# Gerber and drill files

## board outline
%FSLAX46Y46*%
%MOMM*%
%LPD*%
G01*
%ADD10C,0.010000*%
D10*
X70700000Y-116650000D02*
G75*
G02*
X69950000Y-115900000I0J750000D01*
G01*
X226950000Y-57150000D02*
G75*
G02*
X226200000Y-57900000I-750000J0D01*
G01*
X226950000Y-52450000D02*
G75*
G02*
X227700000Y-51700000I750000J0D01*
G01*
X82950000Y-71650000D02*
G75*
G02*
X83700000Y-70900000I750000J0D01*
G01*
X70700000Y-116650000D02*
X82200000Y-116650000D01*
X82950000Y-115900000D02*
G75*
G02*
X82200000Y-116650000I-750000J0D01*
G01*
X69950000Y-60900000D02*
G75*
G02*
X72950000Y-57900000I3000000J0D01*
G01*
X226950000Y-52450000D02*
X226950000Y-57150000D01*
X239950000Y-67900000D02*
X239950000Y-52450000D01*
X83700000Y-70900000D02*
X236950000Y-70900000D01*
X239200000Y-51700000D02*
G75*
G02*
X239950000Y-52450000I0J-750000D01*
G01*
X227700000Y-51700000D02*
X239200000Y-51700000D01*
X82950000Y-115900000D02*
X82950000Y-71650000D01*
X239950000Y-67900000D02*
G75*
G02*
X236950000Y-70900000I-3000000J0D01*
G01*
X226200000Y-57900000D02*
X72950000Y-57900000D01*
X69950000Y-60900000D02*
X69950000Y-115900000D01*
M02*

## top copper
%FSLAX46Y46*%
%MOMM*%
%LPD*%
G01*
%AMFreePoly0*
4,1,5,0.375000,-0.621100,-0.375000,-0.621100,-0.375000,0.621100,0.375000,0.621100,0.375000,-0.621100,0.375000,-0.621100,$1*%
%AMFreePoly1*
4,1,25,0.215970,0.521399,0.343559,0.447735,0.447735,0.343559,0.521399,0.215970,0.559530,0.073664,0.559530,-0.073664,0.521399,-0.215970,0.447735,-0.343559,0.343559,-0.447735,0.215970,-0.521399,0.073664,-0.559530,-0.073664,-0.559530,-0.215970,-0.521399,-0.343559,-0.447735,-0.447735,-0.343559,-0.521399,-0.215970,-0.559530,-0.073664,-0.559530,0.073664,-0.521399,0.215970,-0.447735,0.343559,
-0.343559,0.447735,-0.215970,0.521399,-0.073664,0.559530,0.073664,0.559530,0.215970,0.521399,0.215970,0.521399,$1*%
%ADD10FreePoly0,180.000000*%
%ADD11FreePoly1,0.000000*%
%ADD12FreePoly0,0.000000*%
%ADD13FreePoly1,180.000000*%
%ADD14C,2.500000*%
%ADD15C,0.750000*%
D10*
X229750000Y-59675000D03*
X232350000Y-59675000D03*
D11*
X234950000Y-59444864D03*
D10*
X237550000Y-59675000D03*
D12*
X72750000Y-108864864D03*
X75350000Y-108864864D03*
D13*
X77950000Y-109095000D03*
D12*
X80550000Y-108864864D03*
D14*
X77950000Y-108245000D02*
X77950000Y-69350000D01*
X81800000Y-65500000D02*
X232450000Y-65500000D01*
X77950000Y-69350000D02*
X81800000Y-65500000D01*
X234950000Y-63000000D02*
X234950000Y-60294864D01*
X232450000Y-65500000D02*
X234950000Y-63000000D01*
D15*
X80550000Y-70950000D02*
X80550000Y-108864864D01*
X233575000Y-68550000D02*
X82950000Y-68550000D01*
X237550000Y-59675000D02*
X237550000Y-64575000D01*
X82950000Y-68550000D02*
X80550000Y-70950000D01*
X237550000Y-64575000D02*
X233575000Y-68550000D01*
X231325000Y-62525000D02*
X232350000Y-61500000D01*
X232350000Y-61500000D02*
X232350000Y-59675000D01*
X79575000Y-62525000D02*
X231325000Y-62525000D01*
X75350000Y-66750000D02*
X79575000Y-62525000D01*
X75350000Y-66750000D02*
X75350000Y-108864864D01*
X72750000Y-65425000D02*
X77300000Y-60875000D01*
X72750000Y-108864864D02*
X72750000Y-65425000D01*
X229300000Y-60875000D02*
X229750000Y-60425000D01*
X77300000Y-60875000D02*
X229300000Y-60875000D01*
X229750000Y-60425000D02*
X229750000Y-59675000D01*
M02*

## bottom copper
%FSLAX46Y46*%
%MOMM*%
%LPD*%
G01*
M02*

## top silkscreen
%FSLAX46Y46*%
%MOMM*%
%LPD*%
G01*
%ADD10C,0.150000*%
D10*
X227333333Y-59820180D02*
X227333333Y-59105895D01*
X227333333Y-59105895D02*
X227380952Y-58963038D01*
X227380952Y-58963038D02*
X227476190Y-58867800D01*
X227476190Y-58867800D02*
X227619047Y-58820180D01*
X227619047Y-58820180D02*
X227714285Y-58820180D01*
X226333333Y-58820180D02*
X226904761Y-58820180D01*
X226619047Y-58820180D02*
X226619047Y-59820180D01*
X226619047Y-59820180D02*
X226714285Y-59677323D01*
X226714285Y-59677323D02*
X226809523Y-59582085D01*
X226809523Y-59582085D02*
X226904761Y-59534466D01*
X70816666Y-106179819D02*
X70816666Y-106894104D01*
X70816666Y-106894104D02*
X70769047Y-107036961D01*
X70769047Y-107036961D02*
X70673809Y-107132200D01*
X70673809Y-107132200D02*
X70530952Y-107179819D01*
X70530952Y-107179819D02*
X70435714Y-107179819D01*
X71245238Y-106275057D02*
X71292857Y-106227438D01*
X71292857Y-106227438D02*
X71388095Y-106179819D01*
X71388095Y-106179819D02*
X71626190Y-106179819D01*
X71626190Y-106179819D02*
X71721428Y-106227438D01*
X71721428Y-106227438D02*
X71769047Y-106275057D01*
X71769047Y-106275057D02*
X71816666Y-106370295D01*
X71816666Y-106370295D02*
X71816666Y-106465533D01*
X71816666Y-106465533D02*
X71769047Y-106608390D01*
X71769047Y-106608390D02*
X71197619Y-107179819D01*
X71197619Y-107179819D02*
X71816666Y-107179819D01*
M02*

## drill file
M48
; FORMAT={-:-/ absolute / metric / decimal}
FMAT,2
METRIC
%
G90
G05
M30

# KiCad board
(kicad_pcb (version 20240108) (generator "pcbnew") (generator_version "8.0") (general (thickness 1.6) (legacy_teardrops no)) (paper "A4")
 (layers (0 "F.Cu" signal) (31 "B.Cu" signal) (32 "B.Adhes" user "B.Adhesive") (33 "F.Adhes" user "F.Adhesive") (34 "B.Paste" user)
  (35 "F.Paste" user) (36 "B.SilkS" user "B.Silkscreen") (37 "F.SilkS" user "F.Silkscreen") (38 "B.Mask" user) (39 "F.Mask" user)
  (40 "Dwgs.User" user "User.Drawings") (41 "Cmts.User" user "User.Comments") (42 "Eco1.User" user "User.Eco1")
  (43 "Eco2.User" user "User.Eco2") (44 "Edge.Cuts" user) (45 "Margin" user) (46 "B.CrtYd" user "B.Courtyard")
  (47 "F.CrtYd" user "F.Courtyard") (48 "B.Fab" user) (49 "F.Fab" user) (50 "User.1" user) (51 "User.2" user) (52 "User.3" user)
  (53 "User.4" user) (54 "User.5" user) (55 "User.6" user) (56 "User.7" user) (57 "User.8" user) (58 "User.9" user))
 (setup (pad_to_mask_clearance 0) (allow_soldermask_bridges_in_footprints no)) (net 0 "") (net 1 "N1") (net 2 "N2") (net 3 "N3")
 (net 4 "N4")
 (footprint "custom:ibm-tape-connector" (layer "F.Cu") (at 233.45 56.314864 180)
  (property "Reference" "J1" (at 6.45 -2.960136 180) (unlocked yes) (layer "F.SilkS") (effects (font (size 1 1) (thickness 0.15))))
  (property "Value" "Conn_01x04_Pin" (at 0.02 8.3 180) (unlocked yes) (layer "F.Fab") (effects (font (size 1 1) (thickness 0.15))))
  (pad "1" smd custom (at 3.7 -3.360136 180) (size 0.75 1.2422) (layers "F.Cu" "F.Paste" "F.Mask") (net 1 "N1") (thermal_bridge_angle 45)
   (options (clearance outline) (anchor rect)) (primitives))
  (pad "2" smd custom (at 1.1 -3.360136 180) (size 0.75 1.2422) (layers "F.Cu" "F.Paste" "F.Mask") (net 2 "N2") (thermal_bridge_angle 45)
   (options (clearance outline) (anchor rect)) (primitives))
  (pad "3" smd custom (at -1.5 -3.98) (size 1.128716 1.128716) (drill (offset 0 -0.85)) (layers "F.Cu" "F.Paste" "F.Mask") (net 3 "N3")
   (options (clearance outline) (anchor circle)) (primitives))
  (pad "4" smd custom (at -4.1 -3.360136 180) (size 0.75 1.2422) (layers "F.Cu" "F.Paste" "F.Mask") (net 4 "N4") (thermal_bridge_angle 45)
   (options (clearance outline) (anchor rect)) (primitives)))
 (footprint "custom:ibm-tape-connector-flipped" (layer "F.Cu") (at 76.85 112.225)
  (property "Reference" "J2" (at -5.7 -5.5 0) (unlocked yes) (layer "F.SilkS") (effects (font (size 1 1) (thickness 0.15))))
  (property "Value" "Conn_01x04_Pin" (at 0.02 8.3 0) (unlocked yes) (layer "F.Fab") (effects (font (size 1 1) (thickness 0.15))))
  (pad "1" smd custom (at -4.1 -3.360136) (size 0.75 1.2422) (layers "F.Cu" "F.Paste" "F.Mask") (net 1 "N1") (thermal_bridge_angle 45)
   (options (clearance outline) (anchor rect)) (primitives))
  (pad "2" smd custom (at -1.5 -3.360136) (size 0.75 1.2422) (layers "F.Cu" "F.Paste" "F.Mask") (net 2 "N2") (thermal_bridge_angle 45)
   (options (clearance outline) (anchor rect)) (primitives))
  (pad "3" smd custom (at 1.1 -3.98 180) (size 1.128716 1.128716) (drill (offset 0 -0.85)) (layers "F.Cu" "F.Paste" "F.Mask") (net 3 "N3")
   (options (clearance outline) (anchor circle)) (primitives))
  (pad "4" smd custom (at 3.7 -3.360136) (size 0.75 1.2422) (layers "F.Cu" "F.Paste" "F.Mask") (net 4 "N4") (thermal_bridge_angle 45)
   (options (clearance outline) (anchor rect)) (primitives)))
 (gr_arc (start 70.7 116.65) (mid 70.16967 116.43033) (end 69.95 115.9) (stroke (width 0.01) (type default)) (layer "Edge.Cuts"))
 (gr_arc (start 226.95 57.15) (mid 226.73033 57.68033) (end 226.2 57.9) (stroke (width 0.01) (type default)) (layer "Edge.Cuts"))
 (gr_arc (start 226.95 52.45) (mid 227.16967 51.91967) (end 227.7 51.7) (stroke (width 0.01) (type default)) (layer "Edge.Cuts"))
 (gr_arc (start 82.95 71.65) (mid 83.16967 71.11967) (end 83.7 70.9) (stroke (width 0.01) (type default)) (layer "Edge.Cuts"))
 (gr_line (start 70.7 116.65) (end 82.2 116.65) (stroke (width 0.01) (type default)) (layer "Edge.Cuts"))
 (gr_arc (start 82.95 115.9) (mid 82.73033 116.43033) (end 82.2 116.65) (stroke (width 0.01) (type default)) (layer "Edge.Cuts"))
 (gr_arc (start 69.95 60.9) (mid 70.82868 58.77868) (end 72.95 57.9) (stroke (width 0.01) (type default)) (layer "Edge.Cuts"))
 (gr_line (start 226.95 52.45) (end 226.95 57.15) (stroke (width 0.01) (type default)) (layer "Edge.Cuts"))
 (gr_line (start 239.95 67.9) (end 239.95 52.45) (stroke (width 0.01) (type default)) (layer "Edge.Cuts"))
 (gr_line (start 83.7 70.9) (end 236.95 70.9) (stroke (width 0.01) (type default)) (layer "Edge.Cuts"))
 (gr_arc (start 239.2 51.7) (mid 239.73033 51.91967) (end 239.95 52.45) (stroke (width 0.01) (type default)) (layer "Edge.Cuts"))
 (gr_line (start 227.7 51.7) (end 239.2 51.7) (stroke (width 0.01) (type default)) (layer "Edge.Cuts"))
 (gr_line (start 82.95 115.9) (end 82.95 71.65) (stroke (width 0.01) (type default)) (layer "Edge.Cuts"))
 (gr_arc (start 239.95 67.9) (mid 239.07132 70.02132) (end 236.95 70.9) (stroke (width 0.01) (type default)) (layer "Edge.Cuts"))
 (gr_line (start 226.2 57.9) (end 72.95 57.9) (stroke (width 0.01) (type default)) (layer "Edge.Cuts"))
 (gr_line (start 69.95 60.9) (end 69.95 115.9) (stroke (width 0.01) (type default)) (layer "Edge.Cuts"))
 (segment (start 77.95 108.245) (end 77.95 69.35) (width 2.5) (layer "F.Cu") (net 3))
 (segment (start 81.8 65.5) (end 232.45 65.5) (width 2.5) (layer "F.Cu") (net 3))
 (segment (start 77.95 69.35) (end 81.8 65.5) (width 2.5) (layer "F.Cu") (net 3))
 (segment (start 234.95 63) (end 234.95 60.294864) (width 2.5) (layer "F.Cu") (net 3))
 (segment (start 232.45 65.5) (end 234.95 63) (width 2.5) (layer "F.Cu") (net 3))
 (segment (start 80.55 70.95) (end 80.55 108.864864) (width 0.75) (layer "F.Cu") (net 4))
 (segment (start 233.575 68.55) (end 82.95 68.55) (width 0.75) (layer "F.Cu") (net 4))
 (segment (start 237.55 59.675) (end 237.55 64.575) (width 0.75) (layer "F.Cu") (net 4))
 (segment (start 82.95 68.55) (end 80.55 70.95) (width 0.75) (layer "F.Cu") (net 4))
 (segment (start 237.55 64.575) (end 233.575 68.55) (width 0.75) (layer "F.Cu") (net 4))
 (segment (start 231.325 62.525) (end 232.35 61.5) (width 0.75) (layer "F.Cu") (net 2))
 (segment (start 232.35 61.5) (end 232.35 59.675) (width 0.75) (layer "F.Cu") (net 2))
 (segment (start 79.575 62.525) (end 231.325 62.525) (width 0.75) (layer "F.Cu") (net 2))
 (segment (start 75.35 66.75) (end 79.575 62.525) (width 0.75) (layer "F.Cu") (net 2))
 (segment (start 75.35 66.75) (end 75.35 108.864864) (width 0.75) (layer "F.Cu") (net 2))
 (segment (start 72.75 65.425) (end 77.3 60.875) (width 0.75) (layer "F.Cu") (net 1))
 (segment (start 72.75 108.864864) (end 72.75 65.425) (width 0.75) (layer "F.Cu") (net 1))
 (segment (start 229.3 60.875) (end 229.75 60.425) (width 0.75) (layer "F.Cu") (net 1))
 (segment (start 77.3 60.875) (end 229.3 60.875) (width 0.75) (layer "F.Cu") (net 1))
 (segment (start 229.75 60.425) (end 229.75 59.675) (width 0.75) (layer "F.Cu") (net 1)))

